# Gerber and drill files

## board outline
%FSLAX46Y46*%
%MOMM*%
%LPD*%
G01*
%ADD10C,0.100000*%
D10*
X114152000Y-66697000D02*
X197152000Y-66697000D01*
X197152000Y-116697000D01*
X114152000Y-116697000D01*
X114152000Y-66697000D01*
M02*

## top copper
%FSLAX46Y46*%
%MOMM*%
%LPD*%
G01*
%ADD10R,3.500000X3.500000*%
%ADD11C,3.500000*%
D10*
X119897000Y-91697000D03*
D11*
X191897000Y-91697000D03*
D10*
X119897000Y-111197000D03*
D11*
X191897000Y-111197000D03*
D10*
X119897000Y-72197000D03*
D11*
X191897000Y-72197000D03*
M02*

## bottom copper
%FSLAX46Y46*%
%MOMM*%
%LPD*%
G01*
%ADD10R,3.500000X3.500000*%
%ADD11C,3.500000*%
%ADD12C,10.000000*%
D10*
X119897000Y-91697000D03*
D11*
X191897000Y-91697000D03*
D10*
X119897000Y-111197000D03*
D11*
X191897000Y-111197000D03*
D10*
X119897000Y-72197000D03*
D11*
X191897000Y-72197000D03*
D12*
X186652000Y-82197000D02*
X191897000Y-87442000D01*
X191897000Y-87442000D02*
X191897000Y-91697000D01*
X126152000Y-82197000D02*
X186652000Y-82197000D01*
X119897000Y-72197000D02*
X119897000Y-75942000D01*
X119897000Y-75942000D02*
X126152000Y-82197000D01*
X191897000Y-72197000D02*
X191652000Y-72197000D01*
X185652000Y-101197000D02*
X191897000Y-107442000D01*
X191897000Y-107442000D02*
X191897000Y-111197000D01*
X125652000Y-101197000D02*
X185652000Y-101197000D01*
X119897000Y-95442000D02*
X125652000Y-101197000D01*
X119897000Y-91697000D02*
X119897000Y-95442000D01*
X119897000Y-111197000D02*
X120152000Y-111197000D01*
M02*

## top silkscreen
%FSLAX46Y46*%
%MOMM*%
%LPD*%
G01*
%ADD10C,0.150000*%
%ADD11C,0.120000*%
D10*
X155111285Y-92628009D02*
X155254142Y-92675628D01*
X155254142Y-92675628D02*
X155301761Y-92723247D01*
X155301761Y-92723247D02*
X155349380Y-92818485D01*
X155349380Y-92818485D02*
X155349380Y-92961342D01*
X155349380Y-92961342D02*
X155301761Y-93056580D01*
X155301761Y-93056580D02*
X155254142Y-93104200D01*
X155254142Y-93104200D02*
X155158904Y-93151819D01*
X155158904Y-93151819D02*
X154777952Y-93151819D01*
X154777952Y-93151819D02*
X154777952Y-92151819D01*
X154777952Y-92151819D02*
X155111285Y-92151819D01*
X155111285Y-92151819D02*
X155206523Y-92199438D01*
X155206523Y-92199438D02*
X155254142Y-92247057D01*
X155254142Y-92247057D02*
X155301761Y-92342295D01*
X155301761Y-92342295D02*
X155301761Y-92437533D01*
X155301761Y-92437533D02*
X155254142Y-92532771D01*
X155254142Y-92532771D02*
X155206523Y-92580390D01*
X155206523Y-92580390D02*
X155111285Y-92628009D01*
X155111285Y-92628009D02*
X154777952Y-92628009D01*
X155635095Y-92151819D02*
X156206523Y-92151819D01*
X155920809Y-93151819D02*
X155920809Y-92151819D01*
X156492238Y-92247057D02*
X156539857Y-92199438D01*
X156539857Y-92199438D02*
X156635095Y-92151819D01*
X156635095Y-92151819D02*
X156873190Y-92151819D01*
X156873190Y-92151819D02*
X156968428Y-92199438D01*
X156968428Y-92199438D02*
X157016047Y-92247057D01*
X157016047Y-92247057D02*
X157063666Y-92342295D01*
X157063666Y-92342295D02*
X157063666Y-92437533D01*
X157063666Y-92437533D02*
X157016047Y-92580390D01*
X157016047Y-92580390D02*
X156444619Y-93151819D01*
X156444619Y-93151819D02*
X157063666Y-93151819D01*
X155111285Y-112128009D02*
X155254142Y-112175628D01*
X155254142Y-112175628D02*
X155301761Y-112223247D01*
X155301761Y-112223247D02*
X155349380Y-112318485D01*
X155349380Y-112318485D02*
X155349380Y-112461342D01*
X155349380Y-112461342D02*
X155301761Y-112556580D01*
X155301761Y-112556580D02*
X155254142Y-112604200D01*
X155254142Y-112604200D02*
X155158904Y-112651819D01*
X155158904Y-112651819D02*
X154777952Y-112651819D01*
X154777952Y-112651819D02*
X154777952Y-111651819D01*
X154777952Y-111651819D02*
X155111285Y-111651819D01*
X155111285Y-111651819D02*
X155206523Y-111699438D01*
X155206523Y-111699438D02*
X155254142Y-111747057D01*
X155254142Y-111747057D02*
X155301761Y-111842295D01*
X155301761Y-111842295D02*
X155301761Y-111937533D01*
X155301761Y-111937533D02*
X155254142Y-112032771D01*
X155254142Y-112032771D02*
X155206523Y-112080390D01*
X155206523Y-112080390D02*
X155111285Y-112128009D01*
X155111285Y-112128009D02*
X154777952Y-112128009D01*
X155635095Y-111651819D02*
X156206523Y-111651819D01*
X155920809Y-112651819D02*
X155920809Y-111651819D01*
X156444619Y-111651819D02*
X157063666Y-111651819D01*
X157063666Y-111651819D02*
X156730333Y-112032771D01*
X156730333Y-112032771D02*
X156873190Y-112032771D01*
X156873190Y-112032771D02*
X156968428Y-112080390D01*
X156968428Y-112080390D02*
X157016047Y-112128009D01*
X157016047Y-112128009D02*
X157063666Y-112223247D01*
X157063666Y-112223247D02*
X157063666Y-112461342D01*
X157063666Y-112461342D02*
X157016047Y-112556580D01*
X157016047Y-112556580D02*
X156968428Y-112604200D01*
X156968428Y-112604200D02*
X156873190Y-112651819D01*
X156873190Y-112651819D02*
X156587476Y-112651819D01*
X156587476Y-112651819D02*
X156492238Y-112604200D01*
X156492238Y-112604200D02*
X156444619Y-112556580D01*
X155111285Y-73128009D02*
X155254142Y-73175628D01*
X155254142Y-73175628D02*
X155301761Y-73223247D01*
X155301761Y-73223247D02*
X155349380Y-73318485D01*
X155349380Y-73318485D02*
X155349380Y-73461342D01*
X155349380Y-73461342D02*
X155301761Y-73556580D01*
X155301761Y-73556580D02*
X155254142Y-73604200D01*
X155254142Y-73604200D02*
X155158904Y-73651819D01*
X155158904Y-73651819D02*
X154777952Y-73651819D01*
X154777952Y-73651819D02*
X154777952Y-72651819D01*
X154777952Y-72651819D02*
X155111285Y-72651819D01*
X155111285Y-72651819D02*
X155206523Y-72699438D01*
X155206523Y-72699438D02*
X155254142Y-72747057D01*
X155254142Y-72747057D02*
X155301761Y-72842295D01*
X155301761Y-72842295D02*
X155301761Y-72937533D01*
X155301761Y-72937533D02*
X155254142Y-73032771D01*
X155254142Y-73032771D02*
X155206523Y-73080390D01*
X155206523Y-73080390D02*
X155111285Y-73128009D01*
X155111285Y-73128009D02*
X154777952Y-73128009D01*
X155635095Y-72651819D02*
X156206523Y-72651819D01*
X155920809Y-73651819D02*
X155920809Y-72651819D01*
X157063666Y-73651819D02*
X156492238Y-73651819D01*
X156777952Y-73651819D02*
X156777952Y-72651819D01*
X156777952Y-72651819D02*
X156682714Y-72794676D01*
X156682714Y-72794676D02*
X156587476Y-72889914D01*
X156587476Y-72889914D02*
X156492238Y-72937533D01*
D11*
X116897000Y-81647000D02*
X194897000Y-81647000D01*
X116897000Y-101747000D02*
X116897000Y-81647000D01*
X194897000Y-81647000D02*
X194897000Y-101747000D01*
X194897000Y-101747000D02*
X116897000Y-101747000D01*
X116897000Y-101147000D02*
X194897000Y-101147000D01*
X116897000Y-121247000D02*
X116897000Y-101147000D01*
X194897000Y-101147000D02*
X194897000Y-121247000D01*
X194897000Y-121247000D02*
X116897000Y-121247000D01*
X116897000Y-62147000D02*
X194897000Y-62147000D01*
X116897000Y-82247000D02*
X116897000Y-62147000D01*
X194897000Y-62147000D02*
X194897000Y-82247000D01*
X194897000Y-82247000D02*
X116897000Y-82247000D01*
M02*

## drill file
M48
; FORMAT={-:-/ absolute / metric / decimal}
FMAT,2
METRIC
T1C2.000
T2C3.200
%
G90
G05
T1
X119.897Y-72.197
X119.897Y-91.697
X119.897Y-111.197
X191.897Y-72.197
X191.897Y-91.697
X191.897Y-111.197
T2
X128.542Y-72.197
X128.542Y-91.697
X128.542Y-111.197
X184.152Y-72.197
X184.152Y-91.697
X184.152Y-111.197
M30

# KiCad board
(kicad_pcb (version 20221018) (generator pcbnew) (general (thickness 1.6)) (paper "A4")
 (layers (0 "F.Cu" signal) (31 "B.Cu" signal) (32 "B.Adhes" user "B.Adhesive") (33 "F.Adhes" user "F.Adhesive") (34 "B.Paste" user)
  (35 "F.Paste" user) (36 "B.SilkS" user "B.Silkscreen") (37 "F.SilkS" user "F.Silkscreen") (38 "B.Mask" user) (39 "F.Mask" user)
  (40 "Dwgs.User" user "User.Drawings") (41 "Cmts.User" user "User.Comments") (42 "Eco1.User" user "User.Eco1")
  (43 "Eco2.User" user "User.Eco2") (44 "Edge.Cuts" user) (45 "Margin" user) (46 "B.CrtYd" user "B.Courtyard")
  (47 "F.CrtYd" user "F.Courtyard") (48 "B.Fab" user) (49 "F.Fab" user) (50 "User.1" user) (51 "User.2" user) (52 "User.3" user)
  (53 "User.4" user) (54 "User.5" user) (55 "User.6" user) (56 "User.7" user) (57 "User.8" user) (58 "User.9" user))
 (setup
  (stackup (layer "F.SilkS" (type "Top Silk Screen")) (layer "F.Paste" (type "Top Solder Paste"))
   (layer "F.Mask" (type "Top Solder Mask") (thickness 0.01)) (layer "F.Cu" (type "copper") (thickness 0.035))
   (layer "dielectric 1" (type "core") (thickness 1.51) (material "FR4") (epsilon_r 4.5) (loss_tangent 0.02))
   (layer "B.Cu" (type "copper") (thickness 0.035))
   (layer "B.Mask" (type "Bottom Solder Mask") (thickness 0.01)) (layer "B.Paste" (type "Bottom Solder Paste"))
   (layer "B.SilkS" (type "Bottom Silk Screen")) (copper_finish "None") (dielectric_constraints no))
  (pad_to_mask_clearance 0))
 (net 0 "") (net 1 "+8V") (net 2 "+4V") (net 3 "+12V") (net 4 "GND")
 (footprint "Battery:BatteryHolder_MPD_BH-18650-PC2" (layer "F.Cu") (at 119.897 91.697)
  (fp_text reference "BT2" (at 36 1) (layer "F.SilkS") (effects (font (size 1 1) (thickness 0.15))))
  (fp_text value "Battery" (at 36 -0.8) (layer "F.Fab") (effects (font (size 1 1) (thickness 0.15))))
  (fp_line (start -3 -10.05) (end 75 -10.05) (stroke (width 0.12) (type solid)) (layer "F.SilkS"))
  (fp_line (start -3 10.05) (end -3 -10.05) (stroke (width 0.12) (type solid)) (layer "F.SilkS"))
  (fp_line (start 75 -10.05) (end 75 10.05) (stroke (width 0.12) (type solid)) (layer "F.SilkS"))
  (fp_line (start 75 10.05) (end -3 10.05) (stroke (width 0.12) (type solid)) (layer "F.SilkS"))
  (pad "" np_thru_hole circle (at 8.645 0) (size 3.2 3.2) (drill 3.2) (layers "*.Cu" "*.Mask"))
  (pad "" np_thru_hole circle (at 64.255 0) (size 3.2 3.2) (drill 3.2) (layers "*.Cu" "*.Mask"))
  (pad "1" thru_hole rect (at 0 0) (size 3.5 3.5) (drill 2) (layers "*.Cu" "*.Mask") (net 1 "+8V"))
  (pad "2" thru_hole circle (at 72 0) (size 3.5 3.5) (drill 2) (layers "*.Cu" "*.Mask") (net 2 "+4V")))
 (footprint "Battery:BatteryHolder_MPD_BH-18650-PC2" (layer "F.Cu") (at 119.897 111.197)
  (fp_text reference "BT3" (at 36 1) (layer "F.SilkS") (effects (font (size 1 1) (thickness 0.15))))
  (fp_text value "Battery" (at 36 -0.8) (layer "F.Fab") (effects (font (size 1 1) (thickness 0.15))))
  (fp_line (start -3 -10.05) (end 75 -10.05) (stroke (width 0.12) (type solid)) (layer "F.SilkS"))
  (fp_line (start -3 10.05) (end -3 -10.05) (stroke (width 0.12) (type solid)) (layer "F.SilkS"))
  (fp_line (start 75 -10.05) (end 75 10.05) (stroke (width 0.12) (type solid)) (layer "F.SilkS"))
  (fp_line (start 75 10.05) (end -3 10.05) (stroke (width 0.12) (type solid)) (layer "F.SilkS"))
  (pad "" np_thru_hole circle (at 8.645 0) (size 3.2 3.2) (drill 3.2) (layers "*.Cu" "*.Mask"))
  (pad "" np_thru_hole circle (at 64.255 0) (size 3.2 3.2) (drill 3.2) (layers "*.Cu" "*.Mask"))
  (pad "1" thru_hole rect (at 0 0) (size 3.5 3.5) (drill 2) (layers "*.Cu" "*.Mask") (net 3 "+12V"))
  (pad "2" thru_hole circle (at 72 0) (size 3.5 3.5) (drill 2) (layers "*.Cu" "*.Mask") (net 1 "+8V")))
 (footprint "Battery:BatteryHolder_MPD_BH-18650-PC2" (layer "F.Cu") (at 119.897 72.197)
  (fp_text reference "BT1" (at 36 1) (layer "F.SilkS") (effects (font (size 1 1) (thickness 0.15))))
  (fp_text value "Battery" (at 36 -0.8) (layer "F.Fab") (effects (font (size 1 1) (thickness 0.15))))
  (fp_line (start -3 -10.05) (end 75 -10.05) (stroke (width 0.12) (type solid)) (layer "F.SilkS"))
  (fp_line (start -3 10.05) (end -3 -10.05) (stroke (width 0.12) (type solid)) (layer "F.SilkS"))
  (fp_line (start 75 -10.05) (end 75 10.05) (stroke (width 0.12) (type solid)) (layer "F.SilkS"))
  (fp_line (start 75 10.05) (end -3 10.05) (stroke (width 0.12) (type solid)) (layer "F.SilkS"))
  (pad "" np_thru_hole circle (at 8.645 0) (size 3.2 3.2) (drill 3.2) (layers "*.Cu" "*.Mask"))
  (pad "" np_thru_hole circle (at 64.255 0) (size 3.2 3.2) (drill 3.2) (layers "*.Cu" "*.Mask"))
  (pad "1" thru_hole rect (at 0 0) (size 3.5 3.5) (drill 2) (layers "*.Cu" "*.Mask") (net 2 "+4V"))
  (pad "2" thru_hole circle (at 72 0) (size 3.5 3.5) (drill 2) (layers "*.Cu" "*.Mask") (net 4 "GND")))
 (gr_rect (start 114.152 66.697) (end 197.152 116.697) (stroke (width 0.1) (type default)) (fill none) (layer "Edge.Cuts"))
 (segment (start 186.652 82.197) (end 191.897 87.442) (width 10) (layer "B.Cu") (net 2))
 (segment (start 191.897 87.442) (end 191.897 91.697) (width 10) (layer "B.Cu") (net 2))
 (segment (start 126.152 82.197) (end 186.652 82.197) (width 10) (layer "B.Cu") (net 2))
 (segment (start 119.897 72.197) (end 119.897 75.942) (width 10) (layer "B.Cu") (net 2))
 (segment (start 119.897 75.942) (end 126.152 82.197) (width 10) (layer "B.Cu") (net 2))
 (segment (start 191.897 72.197) (end 191.652 72.197) (width 10) (layer "B.Cu") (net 4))
 (segment (start 185.652 101.197) (end 191.897 107.442) (width 10) (layer "B.Cu") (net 1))
 (segment (start 191.897 107.442) (end 191.897 111.197) (width 10) (layer "B.Cu") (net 1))
 (segment (start 125.652 101.197) (end 185.652 101.197) (width 10) (layer "B.Cu") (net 1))
 (segment (start 119.897 95.442) (end 125.652 101.197) (width 10) (layer "B.Cu") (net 1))
 (segment (start 119.897 91.697) (end 119.897 95.442) (width 10) (layer "B.Cu") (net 1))
 (segment (start 119.897 111.197) (end 120.152 111.197) (width 10) (layer "B.Cu") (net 3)))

